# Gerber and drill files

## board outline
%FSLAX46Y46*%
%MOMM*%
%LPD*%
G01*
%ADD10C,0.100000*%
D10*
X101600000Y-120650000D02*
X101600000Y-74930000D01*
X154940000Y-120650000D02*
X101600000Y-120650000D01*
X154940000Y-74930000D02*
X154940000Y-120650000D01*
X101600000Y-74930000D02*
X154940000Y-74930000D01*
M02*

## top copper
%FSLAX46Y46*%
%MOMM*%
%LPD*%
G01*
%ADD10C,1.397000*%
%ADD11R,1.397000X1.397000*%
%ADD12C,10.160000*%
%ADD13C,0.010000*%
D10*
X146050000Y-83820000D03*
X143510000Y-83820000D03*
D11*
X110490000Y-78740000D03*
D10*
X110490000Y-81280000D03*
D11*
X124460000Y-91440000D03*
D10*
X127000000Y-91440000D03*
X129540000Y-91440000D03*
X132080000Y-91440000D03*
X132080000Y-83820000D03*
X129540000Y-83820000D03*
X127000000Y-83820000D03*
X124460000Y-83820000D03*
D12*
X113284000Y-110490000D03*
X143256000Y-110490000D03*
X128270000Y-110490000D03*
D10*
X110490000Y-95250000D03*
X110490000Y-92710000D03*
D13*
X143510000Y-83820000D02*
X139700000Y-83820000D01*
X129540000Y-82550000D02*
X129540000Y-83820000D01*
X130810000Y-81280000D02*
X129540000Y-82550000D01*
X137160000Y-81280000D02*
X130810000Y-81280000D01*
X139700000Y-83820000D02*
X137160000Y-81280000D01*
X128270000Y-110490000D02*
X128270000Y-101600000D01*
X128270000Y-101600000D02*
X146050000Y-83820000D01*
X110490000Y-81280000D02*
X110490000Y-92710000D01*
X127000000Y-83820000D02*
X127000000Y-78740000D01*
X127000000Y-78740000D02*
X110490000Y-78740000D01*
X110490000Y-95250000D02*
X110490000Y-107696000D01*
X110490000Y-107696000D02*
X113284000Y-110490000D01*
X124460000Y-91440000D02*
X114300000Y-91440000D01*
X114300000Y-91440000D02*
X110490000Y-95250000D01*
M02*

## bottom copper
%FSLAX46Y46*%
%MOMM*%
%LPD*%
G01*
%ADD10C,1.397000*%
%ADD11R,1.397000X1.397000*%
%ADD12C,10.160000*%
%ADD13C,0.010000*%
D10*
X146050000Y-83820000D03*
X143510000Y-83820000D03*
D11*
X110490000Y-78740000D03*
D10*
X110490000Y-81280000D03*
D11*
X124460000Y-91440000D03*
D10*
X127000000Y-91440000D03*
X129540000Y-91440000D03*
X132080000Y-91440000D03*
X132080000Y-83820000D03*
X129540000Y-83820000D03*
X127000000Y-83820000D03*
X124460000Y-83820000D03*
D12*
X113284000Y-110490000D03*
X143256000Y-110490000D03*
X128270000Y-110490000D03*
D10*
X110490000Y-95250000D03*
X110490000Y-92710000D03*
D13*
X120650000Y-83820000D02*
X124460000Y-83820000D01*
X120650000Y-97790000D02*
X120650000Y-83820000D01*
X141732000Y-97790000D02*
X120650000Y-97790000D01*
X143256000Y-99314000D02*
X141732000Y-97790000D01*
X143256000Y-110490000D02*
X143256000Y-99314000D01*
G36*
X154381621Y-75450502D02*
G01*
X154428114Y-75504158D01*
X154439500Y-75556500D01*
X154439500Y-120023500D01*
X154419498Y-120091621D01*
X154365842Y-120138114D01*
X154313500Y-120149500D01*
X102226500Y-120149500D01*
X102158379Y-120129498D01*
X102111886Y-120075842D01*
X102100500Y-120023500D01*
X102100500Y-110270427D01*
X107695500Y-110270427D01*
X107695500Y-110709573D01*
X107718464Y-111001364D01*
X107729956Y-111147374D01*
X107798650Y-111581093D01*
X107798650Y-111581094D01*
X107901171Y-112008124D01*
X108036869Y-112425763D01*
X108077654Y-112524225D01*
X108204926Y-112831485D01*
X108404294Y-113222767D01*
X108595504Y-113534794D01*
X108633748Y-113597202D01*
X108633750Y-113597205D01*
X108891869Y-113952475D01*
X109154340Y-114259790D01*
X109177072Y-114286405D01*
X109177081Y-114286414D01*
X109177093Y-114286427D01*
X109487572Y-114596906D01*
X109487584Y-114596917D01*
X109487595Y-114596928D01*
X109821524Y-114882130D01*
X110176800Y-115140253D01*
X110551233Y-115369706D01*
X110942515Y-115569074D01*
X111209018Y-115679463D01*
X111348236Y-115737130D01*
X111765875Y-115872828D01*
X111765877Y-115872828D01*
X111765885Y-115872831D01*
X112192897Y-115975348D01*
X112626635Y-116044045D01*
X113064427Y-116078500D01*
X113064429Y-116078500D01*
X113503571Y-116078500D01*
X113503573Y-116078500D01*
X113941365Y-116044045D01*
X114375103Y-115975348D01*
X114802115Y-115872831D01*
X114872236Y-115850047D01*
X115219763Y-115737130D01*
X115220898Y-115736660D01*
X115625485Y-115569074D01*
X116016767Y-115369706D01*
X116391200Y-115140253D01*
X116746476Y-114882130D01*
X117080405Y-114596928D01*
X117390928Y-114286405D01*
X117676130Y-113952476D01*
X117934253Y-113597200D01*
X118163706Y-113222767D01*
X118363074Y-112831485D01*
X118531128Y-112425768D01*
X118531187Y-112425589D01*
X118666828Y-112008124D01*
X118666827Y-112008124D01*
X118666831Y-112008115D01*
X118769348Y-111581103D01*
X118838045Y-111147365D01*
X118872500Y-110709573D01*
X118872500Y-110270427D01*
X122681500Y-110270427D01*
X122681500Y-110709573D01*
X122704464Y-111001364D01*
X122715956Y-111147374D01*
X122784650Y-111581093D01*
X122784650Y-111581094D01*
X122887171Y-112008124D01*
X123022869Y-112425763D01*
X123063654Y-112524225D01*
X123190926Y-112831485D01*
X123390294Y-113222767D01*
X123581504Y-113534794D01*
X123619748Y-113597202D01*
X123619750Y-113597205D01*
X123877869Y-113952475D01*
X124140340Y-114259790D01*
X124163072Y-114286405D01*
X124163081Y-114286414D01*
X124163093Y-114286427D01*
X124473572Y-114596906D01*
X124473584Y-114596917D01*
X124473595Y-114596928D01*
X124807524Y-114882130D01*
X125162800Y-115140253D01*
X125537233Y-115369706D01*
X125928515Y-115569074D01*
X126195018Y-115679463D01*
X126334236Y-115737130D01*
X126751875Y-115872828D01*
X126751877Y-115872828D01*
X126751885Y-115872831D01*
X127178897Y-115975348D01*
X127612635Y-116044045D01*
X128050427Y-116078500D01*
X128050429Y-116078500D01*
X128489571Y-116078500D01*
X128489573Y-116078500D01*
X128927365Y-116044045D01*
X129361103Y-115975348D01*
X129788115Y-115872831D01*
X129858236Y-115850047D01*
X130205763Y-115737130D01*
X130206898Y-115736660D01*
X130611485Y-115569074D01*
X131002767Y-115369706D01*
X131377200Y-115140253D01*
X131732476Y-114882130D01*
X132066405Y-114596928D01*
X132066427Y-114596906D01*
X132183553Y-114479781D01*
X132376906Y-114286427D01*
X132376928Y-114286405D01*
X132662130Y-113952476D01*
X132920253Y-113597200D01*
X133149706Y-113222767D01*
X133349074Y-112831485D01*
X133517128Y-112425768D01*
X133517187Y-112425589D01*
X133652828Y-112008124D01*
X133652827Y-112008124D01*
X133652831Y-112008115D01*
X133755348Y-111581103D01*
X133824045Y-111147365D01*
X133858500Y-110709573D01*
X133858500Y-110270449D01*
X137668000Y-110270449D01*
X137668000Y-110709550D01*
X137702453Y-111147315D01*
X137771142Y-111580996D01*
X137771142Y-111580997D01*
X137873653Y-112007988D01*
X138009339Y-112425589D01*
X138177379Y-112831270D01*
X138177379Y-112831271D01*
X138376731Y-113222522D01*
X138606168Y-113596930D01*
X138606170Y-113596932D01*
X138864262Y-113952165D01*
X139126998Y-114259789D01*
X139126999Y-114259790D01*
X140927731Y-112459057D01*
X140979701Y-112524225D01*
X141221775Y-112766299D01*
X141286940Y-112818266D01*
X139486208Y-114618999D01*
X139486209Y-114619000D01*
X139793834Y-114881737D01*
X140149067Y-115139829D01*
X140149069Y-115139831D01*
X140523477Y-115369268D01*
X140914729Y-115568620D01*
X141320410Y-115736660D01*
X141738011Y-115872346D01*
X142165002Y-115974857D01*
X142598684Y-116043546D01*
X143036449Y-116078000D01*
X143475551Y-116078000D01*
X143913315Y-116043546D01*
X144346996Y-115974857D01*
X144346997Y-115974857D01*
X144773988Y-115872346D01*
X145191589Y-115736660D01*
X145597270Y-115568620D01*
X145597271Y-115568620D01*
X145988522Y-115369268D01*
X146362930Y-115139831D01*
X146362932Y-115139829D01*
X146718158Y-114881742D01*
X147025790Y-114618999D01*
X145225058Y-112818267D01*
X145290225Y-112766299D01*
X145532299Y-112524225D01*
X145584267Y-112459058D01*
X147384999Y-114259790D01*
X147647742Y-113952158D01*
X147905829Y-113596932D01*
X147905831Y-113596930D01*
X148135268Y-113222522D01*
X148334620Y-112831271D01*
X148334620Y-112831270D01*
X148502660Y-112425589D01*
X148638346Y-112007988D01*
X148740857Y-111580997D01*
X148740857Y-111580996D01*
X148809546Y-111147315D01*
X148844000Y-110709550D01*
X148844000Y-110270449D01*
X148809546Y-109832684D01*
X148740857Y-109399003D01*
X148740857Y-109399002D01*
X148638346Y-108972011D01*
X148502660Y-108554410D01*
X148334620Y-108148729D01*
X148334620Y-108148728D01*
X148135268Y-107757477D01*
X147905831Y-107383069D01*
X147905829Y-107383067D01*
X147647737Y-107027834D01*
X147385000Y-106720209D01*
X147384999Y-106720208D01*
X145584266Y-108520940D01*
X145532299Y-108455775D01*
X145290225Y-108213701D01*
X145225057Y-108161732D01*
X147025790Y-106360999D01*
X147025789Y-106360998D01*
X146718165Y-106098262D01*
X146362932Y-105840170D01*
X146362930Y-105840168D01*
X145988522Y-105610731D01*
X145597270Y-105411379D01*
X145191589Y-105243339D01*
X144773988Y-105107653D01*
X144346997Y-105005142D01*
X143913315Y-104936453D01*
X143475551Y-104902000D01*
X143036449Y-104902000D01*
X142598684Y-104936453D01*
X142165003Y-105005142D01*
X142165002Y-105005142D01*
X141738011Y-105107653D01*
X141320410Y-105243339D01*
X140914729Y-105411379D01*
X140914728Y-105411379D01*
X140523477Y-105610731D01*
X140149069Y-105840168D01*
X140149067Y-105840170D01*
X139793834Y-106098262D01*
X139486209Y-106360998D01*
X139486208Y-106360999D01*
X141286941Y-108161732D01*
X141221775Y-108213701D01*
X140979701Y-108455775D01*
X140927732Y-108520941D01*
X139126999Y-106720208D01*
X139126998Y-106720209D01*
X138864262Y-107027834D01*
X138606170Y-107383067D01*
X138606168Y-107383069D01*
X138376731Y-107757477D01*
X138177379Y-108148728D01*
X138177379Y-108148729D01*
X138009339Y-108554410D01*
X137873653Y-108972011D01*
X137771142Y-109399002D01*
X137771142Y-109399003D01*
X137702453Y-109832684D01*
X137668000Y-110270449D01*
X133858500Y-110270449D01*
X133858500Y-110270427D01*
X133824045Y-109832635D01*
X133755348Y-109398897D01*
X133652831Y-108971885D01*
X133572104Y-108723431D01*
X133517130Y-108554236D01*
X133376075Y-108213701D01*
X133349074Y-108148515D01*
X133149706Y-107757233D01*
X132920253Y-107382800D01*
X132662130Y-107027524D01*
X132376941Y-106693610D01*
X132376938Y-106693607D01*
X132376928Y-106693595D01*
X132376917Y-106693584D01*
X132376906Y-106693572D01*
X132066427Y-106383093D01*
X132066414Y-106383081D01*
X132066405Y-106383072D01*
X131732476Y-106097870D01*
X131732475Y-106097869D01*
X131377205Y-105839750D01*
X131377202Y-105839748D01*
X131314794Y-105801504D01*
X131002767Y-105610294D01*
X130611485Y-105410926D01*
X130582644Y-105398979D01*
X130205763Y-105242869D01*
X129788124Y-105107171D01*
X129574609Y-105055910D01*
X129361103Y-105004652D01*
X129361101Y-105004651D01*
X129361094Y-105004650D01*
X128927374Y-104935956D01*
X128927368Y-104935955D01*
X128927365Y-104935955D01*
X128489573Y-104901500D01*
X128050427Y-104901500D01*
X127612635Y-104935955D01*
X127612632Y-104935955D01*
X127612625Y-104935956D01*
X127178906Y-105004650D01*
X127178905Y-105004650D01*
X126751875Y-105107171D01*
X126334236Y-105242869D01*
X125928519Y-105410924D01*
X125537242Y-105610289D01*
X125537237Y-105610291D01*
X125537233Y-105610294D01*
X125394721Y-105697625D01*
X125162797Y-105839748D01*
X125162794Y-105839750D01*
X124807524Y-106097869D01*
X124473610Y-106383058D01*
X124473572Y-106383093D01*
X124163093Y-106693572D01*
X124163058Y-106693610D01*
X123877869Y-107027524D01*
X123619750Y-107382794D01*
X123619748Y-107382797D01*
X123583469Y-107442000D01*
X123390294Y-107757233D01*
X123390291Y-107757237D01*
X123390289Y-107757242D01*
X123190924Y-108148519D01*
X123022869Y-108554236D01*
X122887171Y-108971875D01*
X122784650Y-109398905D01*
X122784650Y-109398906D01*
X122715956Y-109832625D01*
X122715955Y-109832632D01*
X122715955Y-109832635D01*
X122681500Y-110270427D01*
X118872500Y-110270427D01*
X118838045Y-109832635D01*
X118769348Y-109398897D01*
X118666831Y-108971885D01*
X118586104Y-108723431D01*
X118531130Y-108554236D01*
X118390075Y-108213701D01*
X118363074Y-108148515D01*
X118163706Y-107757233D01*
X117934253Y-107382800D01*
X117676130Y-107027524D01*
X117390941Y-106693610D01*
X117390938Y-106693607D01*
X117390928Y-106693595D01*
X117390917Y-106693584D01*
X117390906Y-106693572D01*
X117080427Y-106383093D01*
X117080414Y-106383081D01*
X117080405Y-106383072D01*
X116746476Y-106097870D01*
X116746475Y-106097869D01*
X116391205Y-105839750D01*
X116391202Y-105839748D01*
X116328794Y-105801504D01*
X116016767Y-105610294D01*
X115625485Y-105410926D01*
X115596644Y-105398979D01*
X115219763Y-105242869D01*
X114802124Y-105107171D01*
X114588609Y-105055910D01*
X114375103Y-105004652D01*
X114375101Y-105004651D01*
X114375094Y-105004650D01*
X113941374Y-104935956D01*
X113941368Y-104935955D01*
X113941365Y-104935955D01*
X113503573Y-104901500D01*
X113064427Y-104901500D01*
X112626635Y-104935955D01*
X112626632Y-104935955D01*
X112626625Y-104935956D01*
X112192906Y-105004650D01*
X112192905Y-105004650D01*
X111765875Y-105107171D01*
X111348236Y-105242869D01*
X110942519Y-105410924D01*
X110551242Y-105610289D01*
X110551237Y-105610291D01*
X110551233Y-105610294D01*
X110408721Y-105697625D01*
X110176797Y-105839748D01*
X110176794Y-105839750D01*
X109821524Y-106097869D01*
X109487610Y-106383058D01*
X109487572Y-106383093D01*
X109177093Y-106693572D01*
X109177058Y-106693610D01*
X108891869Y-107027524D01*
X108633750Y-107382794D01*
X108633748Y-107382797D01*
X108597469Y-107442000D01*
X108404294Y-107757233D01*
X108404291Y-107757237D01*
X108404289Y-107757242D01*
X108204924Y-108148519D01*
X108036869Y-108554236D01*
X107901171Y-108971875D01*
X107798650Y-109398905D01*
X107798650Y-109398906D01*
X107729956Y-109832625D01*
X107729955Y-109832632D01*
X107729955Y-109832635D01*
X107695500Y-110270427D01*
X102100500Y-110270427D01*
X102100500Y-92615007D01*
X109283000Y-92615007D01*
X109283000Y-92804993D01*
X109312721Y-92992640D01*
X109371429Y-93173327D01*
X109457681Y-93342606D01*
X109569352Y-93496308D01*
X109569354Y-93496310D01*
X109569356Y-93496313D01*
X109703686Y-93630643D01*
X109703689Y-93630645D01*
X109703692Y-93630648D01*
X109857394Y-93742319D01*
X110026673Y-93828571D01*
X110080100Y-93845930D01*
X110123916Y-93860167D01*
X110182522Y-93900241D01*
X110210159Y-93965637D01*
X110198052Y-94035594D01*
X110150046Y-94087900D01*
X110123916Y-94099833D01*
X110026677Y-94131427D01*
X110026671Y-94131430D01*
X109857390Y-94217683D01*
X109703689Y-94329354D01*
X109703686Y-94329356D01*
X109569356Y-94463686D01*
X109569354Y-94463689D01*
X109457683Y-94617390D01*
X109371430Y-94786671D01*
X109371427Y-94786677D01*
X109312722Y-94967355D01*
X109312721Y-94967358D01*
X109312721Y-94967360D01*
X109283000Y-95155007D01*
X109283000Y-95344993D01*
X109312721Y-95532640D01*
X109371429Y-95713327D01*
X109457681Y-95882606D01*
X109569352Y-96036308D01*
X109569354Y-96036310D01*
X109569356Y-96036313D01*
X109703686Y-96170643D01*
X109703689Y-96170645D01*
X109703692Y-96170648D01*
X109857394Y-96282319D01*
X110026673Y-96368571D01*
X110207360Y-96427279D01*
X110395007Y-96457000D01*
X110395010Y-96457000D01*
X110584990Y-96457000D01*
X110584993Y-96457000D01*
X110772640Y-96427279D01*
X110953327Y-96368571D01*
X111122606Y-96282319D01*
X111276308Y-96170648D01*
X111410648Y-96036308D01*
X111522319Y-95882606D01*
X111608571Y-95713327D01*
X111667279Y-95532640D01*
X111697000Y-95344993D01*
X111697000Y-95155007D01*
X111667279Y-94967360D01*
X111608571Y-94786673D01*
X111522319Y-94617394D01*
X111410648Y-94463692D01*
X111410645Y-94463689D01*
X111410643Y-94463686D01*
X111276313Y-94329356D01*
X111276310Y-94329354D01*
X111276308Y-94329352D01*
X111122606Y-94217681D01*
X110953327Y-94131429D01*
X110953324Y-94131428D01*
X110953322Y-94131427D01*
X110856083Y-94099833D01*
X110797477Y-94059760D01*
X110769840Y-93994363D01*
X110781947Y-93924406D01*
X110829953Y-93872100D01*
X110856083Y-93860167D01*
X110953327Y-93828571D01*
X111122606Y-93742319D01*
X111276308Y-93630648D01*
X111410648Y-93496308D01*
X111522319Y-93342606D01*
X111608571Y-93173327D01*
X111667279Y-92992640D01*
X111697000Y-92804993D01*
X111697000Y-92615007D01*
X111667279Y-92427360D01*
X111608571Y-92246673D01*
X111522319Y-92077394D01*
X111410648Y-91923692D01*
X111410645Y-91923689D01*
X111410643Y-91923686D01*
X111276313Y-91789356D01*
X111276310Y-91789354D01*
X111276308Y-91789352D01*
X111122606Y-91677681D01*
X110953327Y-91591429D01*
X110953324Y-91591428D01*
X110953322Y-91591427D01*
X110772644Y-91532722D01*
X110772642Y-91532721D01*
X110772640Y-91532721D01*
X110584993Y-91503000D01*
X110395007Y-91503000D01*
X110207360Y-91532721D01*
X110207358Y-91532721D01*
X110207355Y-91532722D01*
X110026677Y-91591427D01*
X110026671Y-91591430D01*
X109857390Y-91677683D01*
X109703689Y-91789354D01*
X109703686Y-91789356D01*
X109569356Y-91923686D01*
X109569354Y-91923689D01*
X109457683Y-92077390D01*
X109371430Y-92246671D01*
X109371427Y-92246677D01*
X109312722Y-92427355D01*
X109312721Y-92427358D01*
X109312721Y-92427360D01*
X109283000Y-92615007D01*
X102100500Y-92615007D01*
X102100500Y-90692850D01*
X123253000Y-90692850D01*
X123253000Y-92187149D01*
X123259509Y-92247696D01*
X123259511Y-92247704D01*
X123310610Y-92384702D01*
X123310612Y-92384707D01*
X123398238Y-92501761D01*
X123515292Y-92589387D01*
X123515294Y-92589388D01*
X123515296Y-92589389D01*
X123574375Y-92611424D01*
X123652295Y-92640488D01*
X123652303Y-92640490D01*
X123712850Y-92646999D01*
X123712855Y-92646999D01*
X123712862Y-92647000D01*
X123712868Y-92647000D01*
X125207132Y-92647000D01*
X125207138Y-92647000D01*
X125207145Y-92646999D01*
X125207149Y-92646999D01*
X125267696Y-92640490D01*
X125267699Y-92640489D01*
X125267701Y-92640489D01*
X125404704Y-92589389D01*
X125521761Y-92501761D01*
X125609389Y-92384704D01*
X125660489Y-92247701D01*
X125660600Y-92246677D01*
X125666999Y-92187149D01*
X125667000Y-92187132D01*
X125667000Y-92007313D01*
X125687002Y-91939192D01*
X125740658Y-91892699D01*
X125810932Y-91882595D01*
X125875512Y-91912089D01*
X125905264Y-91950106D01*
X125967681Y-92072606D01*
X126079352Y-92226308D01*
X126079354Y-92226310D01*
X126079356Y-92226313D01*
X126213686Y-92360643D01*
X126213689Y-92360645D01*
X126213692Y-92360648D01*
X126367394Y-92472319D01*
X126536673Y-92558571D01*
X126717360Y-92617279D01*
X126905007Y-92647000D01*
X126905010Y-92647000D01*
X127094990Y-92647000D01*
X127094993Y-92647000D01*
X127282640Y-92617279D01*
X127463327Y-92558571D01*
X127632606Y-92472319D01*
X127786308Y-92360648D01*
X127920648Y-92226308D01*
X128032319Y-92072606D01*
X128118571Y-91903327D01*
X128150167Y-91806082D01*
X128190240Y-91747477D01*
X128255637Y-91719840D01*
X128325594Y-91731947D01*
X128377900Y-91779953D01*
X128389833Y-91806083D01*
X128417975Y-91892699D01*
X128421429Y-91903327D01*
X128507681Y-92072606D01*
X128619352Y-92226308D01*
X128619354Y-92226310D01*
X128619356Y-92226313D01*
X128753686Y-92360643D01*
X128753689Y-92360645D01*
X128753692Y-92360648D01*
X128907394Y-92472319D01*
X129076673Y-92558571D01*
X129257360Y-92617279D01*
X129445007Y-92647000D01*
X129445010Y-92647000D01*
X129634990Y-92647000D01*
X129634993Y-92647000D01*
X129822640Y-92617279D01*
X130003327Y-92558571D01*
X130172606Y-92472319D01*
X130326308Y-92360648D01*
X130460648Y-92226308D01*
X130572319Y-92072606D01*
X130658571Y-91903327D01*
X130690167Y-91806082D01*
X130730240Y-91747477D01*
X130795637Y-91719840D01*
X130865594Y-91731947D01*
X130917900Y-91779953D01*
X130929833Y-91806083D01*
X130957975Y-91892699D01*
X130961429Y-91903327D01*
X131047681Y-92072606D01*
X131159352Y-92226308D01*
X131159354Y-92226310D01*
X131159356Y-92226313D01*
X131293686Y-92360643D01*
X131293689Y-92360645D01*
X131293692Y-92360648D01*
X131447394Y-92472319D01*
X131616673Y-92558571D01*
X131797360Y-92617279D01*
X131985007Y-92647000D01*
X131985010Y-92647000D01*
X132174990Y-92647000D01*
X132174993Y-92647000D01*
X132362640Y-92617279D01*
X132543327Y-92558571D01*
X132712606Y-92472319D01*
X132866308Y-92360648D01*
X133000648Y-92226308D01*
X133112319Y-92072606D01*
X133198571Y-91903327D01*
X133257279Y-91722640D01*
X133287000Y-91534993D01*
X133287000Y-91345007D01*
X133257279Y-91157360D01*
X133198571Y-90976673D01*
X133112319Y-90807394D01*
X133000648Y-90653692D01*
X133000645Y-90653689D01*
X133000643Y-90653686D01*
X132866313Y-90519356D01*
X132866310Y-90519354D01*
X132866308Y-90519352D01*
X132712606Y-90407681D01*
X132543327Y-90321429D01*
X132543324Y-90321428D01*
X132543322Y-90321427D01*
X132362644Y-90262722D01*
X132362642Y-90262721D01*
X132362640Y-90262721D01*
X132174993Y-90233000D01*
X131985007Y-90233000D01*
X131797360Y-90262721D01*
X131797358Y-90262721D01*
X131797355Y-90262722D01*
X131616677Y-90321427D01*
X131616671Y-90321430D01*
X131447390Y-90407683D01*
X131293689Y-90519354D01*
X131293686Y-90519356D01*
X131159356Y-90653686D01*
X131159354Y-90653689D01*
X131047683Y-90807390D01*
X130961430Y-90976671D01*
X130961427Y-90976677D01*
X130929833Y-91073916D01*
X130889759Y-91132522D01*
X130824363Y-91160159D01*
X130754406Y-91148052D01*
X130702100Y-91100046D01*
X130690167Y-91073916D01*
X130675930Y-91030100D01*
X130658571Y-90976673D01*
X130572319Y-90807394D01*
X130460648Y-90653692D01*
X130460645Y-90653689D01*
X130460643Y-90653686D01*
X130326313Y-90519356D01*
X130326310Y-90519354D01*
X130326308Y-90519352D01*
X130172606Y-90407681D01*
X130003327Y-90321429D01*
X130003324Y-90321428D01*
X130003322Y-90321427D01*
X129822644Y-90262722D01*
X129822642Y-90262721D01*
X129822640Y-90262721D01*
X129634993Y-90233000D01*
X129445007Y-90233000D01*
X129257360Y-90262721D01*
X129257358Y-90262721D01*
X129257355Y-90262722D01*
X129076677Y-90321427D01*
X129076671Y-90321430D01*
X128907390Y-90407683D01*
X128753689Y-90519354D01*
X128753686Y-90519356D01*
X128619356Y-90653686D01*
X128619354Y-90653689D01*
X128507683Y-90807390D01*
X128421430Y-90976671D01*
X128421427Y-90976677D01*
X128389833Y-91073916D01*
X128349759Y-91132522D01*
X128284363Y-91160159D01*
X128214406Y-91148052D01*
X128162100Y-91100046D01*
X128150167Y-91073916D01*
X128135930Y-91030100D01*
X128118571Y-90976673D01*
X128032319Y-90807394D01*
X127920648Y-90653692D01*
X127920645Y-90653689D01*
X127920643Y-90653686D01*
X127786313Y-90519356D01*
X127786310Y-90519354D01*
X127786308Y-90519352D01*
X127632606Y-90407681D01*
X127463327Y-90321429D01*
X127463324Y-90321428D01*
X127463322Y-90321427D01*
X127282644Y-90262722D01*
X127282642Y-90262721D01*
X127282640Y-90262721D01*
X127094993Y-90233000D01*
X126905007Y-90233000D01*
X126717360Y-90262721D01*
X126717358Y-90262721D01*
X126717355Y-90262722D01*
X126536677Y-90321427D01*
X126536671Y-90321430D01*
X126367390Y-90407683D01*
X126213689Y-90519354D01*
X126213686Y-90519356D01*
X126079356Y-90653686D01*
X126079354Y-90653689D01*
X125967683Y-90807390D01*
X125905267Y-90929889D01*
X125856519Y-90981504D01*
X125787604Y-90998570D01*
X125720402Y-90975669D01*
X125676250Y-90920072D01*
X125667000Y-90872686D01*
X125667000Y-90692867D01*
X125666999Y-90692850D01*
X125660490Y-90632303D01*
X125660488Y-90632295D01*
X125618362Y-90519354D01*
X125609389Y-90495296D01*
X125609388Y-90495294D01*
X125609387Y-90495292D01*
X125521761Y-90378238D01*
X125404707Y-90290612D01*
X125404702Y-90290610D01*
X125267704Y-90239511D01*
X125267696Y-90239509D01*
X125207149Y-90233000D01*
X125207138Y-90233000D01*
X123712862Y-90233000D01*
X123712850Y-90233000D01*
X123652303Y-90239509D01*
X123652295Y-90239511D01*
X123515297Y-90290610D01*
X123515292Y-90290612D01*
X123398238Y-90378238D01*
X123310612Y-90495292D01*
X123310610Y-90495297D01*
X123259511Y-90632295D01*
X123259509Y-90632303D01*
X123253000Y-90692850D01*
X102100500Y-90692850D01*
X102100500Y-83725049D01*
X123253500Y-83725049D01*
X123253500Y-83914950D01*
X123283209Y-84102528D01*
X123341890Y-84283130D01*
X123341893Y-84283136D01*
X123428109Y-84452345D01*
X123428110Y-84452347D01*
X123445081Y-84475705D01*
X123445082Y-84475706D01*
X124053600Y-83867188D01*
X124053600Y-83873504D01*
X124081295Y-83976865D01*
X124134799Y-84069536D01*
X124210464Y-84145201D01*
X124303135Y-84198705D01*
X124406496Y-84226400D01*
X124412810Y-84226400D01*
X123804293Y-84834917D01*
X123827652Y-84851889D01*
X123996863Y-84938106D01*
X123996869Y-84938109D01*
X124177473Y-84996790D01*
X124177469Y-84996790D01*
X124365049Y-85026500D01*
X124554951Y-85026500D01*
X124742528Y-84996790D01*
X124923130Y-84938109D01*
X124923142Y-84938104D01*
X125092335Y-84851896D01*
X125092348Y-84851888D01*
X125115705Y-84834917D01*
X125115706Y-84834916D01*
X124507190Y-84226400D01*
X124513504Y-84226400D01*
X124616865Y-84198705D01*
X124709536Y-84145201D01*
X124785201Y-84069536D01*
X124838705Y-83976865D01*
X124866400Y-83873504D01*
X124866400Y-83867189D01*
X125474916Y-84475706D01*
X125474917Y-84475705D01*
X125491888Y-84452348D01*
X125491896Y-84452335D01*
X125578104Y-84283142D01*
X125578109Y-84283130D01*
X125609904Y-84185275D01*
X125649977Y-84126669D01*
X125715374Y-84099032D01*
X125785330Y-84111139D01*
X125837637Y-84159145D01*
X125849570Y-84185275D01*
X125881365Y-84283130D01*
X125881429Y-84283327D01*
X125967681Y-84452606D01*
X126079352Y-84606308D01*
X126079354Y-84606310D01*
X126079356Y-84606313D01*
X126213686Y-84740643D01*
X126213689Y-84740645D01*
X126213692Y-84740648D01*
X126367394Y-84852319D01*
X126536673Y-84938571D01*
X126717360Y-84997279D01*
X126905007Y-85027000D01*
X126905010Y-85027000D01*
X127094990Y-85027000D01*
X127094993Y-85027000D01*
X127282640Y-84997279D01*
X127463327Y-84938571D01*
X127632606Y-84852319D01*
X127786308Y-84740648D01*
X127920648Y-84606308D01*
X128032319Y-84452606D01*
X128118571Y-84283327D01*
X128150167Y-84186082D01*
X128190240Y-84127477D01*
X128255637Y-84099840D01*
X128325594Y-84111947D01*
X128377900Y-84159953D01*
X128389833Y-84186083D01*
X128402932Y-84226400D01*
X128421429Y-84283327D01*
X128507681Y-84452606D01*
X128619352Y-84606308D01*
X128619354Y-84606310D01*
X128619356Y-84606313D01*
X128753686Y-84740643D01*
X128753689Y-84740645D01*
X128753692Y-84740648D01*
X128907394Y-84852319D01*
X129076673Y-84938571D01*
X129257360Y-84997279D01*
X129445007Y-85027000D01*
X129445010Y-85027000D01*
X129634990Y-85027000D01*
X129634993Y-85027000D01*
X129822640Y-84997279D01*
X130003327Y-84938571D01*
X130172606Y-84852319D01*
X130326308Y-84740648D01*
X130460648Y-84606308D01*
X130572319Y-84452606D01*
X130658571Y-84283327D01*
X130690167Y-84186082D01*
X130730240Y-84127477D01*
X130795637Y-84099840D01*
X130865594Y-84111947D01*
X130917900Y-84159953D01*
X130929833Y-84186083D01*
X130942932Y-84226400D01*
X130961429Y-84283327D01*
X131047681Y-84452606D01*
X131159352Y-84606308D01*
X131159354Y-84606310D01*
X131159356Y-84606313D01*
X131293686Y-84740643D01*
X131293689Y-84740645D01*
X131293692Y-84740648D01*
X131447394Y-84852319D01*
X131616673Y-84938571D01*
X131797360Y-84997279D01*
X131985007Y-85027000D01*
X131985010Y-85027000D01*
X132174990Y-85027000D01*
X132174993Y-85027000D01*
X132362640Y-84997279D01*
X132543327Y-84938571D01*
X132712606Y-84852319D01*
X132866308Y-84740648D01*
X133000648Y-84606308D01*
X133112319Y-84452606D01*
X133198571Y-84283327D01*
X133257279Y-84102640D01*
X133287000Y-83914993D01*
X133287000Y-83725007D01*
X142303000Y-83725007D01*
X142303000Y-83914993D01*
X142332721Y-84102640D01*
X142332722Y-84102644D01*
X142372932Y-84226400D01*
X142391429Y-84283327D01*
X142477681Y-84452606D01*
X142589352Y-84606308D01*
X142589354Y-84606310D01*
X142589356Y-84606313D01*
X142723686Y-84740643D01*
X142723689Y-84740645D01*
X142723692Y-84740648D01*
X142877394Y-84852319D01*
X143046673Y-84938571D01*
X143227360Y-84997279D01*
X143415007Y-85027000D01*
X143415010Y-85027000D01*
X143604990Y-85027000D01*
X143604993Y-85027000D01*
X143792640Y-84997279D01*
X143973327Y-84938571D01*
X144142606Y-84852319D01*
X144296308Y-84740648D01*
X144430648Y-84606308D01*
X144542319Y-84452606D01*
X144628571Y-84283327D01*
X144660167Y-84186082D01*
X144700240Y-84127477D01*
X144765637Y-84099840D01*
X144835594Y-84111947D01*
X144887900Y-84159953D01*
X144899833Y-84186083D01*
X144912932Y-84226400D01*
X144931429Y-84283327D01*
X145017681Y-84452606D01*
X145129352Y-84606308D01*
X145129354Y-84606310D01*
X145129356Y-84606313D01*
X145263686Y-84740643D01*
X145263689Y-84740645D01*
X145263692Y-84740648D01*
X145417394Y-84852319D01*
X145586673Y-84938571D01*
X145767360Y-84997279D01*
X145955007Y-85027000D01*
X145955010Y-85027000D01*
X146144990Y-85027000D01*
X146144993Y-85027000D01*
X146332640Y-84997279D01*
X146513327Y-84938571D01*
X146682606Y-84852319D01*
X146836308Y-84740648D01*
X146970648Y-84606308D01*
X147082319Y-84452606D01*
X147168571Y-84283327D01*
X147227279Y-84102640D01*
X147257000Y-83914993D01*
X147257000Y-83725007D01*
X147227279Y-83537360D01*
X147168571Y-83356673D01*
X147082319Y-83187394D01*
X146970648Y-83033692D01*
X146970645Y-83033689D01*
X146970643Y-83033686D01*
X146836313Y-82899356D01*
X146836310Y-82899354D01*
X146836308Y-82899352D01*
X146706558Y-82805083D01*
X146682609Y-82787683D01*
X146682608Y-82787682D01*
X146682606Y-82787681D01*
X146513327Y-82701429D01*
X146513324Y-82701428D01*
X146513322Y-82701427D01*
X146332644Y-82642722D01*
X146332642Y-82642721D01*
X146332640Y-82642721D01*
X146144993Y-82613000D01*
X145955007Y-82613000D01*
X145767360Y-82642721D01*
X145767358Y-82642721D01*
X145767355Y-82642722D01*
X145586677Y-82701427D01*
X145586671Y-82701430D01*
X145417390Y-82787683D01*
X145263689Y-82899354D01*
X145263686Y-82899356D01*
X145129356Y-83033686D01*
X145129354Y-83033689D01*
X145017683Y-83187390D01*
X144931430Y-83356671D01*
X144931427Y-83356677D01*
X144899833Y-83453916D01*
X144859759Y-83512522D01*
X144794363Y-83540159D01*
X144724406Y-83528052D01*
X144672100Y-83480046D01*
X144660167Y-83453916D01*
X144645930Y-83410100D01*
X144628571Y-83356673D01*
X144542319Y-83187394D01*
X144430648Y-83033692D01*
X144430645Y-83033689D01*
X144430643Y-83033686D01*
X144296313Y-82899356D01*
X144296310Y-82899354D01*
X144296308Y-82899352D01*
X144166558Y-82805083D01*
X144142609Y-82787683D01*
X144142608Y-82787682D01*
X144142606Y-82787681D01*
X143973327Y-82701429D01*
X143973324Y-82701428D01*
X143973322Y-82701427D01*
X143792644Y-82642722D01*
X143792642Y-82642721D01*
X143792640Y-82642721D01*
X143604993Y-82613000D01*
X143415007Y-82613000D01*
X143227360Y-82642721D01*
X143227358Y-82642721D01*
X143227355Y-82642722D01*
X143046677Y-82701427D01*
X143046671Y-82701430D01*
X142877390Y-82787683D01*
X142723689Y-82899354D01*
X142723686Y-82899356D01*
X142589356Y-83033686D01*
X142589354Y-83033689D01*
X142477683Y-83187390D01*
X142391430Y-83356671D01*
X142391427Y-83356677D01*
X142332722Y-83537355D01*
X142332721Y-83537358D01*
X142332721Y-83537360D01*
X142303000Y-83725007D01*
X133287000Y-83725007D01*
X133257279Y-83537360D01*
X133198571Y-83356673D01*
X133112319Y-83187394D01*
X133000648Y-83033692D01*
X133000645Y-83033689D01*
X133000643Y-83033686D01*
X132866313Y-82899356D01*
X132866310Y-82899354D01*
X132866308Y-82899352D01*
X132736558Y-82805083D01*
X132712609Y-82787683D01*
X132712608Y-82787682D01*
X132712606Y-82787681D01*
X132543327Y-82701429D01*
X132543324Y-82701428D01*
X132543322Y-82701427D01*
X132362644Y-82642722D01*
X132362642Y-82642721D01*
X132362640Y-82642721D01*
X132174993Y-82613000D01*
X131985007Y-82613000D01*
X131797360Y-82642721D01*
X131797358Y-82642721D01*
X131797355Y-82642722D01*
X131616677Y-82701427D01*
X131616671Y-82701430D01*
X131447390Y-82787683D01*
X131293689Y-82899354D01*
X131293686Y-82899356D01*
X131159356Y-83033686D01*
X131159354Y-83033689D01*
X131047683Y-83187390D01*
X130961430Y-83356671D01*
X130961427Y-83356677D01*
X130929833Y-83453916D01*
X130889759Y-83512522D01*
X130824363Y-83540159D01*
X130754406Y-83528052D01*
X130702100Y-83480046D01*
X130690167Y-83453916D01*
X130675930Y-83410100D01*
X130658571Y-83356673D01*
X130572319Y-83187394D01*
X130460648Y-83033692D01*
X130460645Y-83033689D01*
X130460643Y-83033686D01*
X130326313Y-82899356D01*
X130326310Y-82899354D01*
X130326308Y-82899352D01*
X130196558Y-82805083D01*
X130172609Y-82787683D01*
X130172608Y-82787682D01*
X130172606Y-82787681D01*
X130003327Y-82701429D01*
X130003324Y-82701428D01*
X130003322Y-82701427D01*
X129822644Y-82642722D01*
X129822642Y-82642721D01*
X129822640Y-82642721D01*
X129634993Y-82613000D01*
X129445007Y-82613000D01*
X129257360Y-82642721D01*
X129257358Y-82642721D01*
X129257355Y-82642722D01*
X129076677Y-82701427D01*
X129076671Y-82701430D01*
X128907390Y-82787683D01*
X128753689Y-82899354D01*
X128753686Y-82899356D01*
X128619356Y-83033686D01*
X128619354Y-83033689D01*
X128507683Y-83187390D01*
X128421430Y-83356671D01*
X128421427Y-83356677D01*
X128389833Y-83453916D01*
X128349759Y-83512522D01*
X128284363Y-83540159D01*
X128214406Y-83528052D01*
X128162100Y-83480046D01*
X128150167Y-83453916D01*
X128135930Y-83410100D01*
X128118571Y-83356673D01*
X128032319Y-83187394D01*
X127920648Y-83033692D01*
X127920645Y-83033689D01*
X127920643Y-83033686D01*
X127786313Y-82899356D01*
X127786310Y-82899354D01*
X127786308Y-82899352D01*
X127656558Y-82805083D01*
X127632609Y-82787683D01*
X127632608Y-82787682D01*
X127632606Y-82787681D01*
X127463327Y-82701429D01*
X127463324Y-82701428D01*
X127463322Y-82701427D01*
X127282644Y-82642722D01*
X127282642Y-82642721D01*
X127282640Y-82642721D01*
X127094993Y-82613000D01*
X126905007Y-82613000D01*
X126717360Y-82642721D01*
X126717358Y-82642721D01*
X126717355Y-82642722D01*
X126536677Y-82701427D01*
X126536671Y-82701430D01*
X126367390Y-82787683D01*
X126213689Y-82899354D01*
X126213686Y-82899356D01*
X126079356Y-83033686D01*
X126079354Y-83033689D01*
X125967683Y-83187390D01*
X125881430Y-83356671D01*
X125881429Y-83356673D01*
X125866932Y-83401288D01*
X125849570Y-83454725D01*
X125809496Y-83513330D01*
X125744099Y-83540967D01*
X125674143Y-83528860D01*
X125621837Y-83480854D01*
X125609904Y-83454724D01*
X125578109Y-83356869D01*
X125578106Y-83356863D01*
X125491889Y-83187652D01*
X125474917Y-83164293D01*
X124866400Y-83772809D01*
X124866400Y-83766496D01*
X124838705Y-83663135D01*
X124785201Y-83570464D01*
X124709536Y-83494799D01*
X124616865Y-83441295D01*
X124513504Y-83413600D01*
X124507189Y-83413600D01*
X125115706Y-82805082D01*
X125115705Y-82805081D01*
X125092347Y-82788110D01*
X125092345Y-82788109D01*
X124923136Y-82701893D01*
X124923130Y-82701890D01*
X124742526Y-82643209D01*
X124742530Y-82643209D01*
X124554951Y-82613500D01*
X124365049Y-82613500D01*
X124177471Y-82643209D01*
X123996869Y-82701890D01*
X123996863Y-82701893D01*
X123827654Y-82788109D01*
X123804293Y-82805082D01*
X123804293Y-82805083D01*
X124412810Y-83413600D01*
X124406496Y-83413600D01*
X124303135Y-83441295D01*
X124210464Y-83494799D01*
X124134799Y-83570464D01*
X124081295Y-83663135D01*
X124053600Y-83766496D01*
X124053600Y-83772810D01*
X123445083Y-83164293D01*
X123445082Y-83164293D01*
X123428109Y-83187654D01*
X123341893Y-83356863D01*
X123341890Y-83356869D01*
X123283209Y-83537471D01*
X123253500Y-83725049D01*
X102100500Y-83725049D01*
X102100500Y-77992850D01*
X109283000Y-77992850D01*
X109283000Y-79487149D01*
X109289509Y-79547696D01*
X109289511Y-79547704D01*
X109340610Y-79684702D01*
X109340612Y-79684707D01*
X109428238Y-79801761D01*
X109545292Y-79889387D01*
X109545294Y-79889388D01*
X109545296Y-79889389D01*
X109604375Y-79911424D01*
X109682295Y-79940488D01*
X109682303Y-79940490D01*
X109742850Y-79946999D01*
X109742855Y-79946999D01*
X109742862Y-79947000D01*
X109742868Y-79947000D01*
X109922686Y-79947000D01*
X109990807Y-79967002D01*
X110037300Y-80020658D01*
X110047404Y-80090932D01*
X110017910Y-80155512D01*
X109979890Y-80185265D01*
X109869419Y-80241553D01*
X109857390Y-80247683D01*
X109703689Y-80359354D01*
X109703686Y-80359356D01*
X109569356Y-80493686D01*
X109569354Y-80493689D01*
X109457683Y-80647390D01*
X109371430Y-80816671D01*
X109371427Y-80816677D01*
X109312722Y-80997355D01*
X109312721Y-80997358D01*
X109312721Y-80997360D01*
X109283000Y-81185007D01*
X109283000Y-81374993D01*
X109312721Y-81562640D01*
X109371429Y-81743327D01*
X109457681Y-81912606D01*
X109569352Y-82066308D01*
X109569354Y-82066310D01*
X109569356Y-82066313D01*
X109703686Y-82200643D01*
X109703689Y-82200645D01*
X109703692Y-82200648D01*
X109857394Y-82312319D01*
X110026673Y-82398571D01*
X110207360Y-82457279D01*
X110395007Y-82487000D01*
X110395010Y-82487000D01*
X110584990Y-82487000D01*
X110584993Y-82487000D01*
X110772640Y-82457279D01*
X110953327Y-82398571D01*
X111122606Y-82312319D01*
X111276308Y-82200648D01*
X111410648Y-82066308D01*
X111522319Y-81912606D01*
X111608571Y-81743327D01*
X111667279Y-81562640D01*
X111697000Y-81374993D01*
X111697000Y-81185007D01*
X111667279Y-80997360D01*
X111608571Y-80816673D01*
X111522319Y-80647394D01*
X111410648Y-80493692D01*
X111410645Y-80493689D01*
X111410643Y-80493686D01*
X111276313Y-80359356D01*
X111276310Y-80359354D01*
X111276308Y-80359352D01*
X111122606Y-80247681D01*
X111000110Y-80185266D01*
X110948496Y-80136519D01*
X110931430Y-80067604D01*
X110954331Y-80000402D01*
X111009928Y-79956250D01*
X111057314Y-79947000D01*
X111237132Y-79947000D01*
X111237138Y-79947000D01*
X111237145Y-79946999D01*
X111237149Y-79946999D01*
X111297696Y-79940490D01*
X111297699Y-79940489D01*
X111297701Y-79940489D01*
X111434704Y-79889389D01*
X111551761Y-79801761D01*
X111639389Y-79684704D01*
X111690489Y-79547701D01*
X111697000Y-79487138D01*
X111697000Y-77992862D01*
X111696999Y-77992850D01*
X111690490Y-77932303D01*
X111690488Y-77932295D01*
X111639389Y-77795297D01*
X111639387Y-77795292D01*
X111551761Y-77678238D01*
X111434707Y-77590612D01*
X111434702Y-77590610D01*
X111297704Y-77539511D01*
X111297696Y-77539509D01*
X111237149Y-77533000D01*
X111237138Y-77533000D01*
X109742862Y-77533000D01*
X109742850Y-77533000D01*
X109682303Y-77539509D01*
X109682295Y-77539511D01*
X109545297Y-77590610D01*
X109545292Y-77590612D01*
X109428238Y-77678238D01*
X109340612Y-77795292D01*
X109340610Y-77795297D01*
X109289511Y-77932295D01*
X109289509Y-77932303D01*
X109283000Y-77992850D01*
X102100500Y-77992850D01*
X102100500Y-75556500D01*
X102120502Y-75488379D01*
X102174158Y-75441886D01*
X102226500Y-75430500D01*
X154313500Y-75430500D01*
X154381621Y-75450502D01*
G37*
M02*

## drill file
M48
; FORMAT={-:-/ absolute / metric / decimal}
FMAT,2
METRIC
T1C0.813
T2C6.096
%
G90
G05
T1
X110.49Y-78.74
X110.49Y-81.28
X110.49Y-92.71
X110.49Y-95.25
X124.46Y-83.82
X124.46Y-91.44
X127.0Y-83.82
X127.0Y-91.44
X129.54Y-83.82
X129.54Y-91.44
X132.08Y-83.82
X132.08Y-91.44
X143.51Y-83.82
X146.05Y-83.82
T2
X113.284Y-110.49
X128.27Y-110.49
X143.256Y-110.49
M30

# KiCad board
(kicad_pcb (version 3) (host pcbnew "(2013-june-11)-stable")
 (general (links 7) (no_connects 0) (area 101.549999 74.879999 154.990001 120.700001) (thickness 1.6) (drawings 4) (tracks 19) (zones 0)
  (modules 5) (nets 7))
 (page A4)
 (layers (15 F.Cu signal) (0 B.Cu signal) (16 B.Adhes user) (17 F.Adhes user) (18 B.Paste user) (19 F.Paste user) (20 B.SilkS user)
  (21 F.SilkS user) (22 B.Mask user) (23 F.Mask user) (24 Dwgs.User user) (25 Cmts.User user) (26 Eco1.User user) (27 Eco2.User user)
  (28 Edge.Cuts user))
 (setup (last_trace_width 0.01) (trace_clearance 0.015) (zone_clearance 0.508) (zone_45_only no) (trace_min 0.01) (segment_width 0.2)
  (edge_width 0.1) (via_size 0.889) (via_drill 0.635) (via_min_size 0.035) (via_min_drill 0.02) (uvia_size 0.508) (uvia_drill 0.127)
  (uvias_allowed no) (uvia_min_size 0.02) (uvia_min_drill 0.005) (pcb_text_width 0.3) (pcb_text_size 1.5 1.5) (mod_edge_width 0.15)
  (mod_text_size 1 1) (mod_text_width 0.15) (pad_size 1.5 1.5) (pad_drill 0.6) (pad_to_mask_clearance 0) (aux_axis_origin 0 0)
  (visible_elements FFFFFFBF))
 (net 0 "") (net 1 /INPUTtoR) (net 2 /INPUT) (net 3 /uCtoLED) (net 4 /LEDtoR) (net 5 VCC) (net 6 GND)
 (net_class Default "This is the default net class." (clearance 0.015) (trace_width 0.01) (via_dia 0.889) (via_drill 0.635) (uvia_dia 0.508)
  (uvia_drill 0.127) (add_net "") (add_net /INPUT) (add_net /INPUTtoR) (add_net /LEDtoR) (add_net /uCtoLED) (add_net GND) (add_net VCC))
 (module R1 (layer F.Cu) (at 144.78 83.82 180) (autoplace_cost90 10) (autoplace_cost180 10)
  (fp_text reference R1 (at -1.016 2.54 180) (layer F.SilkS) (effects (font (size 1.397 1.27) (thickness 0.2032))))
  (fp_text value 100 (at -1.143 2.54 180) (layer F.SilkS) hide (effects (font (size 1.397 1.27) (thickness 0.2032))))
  (pad 1 thru_hole circle (at -1.27 0 180) (size 1.397 1.397) (drill 0.8128) (layers *.Cu *.Mask F.SilkS) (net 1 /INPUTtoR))
  (pad 2 thru_hole circle (at 1.27 0 180) (size 1.397 1.397) (drill 0.8128) (layers *.Cu *.Mask F.SilkS) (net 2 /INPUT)))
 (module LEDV (layer F.Cu) (at 110.49 80.01 270)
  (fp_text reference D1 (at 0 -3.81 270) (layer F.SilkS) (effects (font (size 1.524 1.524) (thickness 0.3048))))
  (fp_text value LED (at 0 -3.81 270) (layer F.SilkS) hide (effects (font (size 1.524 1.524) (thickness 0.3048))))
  (pad 1 thru_hole rect (at -1.27 0 270) (size 1.397 1.397) (drill 0.8128) (layers *.Cu *.Mask F.SilkS) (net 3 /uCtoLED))
  (pad 2 thru_hole circle (at 1.27 0 270) (size 1.397 1.397) (drill 0.8128) (layers *.Cu *.Mask F.SilkS) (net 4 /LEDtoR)))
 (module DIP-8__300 (layer F.Cu) (at 128.27 87.63)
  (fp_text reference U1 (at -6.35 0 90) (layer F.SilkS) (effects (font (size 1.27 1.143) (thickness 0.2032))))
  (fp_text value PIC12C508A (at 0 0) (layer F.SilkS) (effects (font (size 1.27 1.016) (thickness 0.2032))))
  (pad 1 thru_hole rect (at -3.81 3.81) (size 1.397 1.397) (drill 0.8128) (layers *.Cu *.Mask F.SilkS) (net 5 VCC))
  (pad 2 thru_hole circle (at -1.27 3.81) (size 1.397 1.397) (drill 0.8128) (layers *.Cu *.Mask F.SilkS))
  (pad 3 thru_hole circle (at 1.27 3.81) (size 1.397 1.397) (drill 0.8128) (layers *.Cu *.Mask F.SilkS))
  (pad 4 thru_hole circle (at 3.81 3.81) (size 1.397 1.397) (drill 0.8128) (layers *.Cu *.Mask F.SilkS))
  (pad 5 thru_hole circle (at 3.81 -3.81) (size 1.397 1.397) (drill 0.8128) (layers *.Cu *.Mask F.SilkS))
  (pad 6 thru_hole circle (at 1.27 -3.81) (size 1.397 1.397) (drill 0.8128) (layers *.Cu *.Mask F.SilkS) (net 2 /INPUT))
  (pad 7 thru_hole circle (at -1.27 -3.81) (size 1.397 1.397) (drill 0.8128) (layers *.Cu *.Mask F.SilkS) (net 3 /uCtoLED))
  (pad 8 thru_hole circle (at -3.81 -3.81) (size 1.397 1.397) (drill 0.8128) (layers *.Cu *.Mask F.SilkS) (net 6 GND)))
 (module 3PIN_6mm (layer F.Cu) (at 128.27 110.49)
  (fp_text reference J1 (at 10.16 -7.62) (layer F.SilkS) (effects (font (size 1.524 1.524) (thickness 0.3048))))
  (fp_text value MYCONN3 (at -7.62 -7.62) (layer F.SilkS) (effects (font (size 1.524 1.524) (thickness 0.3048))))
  (pad 1 thru_hole circle (at -14.986 0) (size 10.16 10.16) (drill 6.096) (layers *.Cu *.Mask F.SilkS) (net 5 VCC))
  (pad 3 thru_hole circle (at 14.986 0) (size 10.16 10.16) (drill 6.096) (layers *.Cu *.Mask F.SilkS) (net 6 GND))
  (pad 2 thru_hole circle (at 0 0) (size 10.16 10.16) (drill 6.096) (layers *.Cu *.Mask F.SilkS) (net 1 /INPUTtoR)))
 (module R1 (layer F.Cu) (at 110.49 93.98 90) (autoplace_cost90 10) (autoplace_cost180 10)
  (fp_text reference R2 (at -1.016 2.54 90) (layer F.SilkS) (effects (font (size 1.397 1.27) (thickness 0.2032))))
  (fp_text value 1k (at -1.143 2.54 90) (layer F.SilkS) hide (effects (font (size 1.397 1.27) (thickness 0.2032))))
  (pad 1 thru_hole circle (at -1.27 0 90) (size 1.397 1.397) (drill 0.8128) (layers *.Cu *.Mask F.SilkS) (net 5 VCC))
  (pad 2 thru_hole circle (at 1.27 0 90) (size 1.397 1.397) (drill 0.8128) (layers *.Cu *.Mask F.SilkS) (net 4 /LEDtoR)))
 (gr_line (start 101.6 120.65) (end 101.6 74.93) (angle 90) (layer Edge.Cuts) (width 0.1))
 (gr_line (start 154.94 120.65) (end 101.6 120.65) (angle 90) (layer Edge.Cuts) (width 0.1))
 (gr_line (start 154.94 74.93) (end 154.94 120.65) (angle 90) (layer Edge.Cuts) (width 0.1))
 (gr_line (start 101.6 74.93) (end 154.94 74.93) (angle 90) (layer Edge.Cuts) (width 0.1))
 (segment (start 143.51 83.82) (end 139.7 83.82) (width 0.01) (layer F.Cu) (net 2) (status 10))
 (segment (start 129.54 82.55) (end 129.54 83.82) (width 0.01) (layer F.Cu) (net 2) (status 20))
 (segment (start 130.81 81.28) (end 129.54 82.55) (width 0.01) (layer F.Cu) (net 2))
 (segment (start 137.16 81.28) (end 130.81 81.28) (width 0.01) (layer F.Cu) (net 2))
 (segment (start 139.7 83.82) (end 137.16 81.28) (width 0.01) (layer F.Cu) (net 2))
 (segment (start 128.27 110.49) (end 128.27 101.6) (width 0.01) (layer F.Cu) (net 1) (status 10))
 (segment (start 128.27 101.6) (end 146.05 83.82) (width 0.01) (layer F.Cu) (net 1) (status 20))
 (segment (start 110.49 81.28) (end 110.49 92.71) (width 0.01) (layer F.Cu) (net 4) (status 30))
 (segment (start 127 83.82) (end 127 78.74) (width 0.01) (layer F.Cu) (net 3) (status 10))
 (segment (start 127 78.74) (end 110.49 78.74) (width 0.01) (layer F.Cu) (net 3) (status 20))
 (segment (start 120.65 83.82) (end 124.46 83.82) (width 0.01) (layer B.Cu) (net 6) (status 20))
 (segment (start 120.65 97.79) (end 120.65 83.82) (width 0.01) (layer B.Cu) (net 6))
 (segment (start 141.732 97.79) (end 120.65 97.79) (width 0.01) (layer B.Cu) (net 6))
 (segment (start 143.256 99.314) (end 141.732 97.79) (width 0.01) (layer B.Cu) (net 6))
 (segment (start 143.256 110.49) (end 143.256 99.314) (width 0.01) (layer B.Cu) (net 6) (status 10))
 (segment (start 110.49 95.25) (end 110.49 107.696) (width 0.01) (layer F.Cu) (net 5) (status 30))
 (segment (start 110.49 107.696) (end 113.284 110.49) (width 0.01) (layer F.Cu) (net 5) (status 30))
 (segment (start 124.46 91.44) (end 114.3 91.44) (width 0.01) (layer F.Cu) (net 5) (status 10))
 (segment (start 114.3 91.44) (end 110.49 95.25) (width 0.01) (layer F.Cu) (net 5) (status 20))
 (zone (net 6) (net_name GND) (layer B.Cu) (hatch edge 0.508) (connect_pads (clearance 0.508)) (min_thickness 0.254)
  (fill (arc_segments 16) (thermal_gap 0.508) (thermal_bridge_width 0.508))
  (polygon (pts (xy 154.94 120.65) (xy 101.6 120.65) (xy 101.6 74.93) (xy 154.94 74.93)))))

